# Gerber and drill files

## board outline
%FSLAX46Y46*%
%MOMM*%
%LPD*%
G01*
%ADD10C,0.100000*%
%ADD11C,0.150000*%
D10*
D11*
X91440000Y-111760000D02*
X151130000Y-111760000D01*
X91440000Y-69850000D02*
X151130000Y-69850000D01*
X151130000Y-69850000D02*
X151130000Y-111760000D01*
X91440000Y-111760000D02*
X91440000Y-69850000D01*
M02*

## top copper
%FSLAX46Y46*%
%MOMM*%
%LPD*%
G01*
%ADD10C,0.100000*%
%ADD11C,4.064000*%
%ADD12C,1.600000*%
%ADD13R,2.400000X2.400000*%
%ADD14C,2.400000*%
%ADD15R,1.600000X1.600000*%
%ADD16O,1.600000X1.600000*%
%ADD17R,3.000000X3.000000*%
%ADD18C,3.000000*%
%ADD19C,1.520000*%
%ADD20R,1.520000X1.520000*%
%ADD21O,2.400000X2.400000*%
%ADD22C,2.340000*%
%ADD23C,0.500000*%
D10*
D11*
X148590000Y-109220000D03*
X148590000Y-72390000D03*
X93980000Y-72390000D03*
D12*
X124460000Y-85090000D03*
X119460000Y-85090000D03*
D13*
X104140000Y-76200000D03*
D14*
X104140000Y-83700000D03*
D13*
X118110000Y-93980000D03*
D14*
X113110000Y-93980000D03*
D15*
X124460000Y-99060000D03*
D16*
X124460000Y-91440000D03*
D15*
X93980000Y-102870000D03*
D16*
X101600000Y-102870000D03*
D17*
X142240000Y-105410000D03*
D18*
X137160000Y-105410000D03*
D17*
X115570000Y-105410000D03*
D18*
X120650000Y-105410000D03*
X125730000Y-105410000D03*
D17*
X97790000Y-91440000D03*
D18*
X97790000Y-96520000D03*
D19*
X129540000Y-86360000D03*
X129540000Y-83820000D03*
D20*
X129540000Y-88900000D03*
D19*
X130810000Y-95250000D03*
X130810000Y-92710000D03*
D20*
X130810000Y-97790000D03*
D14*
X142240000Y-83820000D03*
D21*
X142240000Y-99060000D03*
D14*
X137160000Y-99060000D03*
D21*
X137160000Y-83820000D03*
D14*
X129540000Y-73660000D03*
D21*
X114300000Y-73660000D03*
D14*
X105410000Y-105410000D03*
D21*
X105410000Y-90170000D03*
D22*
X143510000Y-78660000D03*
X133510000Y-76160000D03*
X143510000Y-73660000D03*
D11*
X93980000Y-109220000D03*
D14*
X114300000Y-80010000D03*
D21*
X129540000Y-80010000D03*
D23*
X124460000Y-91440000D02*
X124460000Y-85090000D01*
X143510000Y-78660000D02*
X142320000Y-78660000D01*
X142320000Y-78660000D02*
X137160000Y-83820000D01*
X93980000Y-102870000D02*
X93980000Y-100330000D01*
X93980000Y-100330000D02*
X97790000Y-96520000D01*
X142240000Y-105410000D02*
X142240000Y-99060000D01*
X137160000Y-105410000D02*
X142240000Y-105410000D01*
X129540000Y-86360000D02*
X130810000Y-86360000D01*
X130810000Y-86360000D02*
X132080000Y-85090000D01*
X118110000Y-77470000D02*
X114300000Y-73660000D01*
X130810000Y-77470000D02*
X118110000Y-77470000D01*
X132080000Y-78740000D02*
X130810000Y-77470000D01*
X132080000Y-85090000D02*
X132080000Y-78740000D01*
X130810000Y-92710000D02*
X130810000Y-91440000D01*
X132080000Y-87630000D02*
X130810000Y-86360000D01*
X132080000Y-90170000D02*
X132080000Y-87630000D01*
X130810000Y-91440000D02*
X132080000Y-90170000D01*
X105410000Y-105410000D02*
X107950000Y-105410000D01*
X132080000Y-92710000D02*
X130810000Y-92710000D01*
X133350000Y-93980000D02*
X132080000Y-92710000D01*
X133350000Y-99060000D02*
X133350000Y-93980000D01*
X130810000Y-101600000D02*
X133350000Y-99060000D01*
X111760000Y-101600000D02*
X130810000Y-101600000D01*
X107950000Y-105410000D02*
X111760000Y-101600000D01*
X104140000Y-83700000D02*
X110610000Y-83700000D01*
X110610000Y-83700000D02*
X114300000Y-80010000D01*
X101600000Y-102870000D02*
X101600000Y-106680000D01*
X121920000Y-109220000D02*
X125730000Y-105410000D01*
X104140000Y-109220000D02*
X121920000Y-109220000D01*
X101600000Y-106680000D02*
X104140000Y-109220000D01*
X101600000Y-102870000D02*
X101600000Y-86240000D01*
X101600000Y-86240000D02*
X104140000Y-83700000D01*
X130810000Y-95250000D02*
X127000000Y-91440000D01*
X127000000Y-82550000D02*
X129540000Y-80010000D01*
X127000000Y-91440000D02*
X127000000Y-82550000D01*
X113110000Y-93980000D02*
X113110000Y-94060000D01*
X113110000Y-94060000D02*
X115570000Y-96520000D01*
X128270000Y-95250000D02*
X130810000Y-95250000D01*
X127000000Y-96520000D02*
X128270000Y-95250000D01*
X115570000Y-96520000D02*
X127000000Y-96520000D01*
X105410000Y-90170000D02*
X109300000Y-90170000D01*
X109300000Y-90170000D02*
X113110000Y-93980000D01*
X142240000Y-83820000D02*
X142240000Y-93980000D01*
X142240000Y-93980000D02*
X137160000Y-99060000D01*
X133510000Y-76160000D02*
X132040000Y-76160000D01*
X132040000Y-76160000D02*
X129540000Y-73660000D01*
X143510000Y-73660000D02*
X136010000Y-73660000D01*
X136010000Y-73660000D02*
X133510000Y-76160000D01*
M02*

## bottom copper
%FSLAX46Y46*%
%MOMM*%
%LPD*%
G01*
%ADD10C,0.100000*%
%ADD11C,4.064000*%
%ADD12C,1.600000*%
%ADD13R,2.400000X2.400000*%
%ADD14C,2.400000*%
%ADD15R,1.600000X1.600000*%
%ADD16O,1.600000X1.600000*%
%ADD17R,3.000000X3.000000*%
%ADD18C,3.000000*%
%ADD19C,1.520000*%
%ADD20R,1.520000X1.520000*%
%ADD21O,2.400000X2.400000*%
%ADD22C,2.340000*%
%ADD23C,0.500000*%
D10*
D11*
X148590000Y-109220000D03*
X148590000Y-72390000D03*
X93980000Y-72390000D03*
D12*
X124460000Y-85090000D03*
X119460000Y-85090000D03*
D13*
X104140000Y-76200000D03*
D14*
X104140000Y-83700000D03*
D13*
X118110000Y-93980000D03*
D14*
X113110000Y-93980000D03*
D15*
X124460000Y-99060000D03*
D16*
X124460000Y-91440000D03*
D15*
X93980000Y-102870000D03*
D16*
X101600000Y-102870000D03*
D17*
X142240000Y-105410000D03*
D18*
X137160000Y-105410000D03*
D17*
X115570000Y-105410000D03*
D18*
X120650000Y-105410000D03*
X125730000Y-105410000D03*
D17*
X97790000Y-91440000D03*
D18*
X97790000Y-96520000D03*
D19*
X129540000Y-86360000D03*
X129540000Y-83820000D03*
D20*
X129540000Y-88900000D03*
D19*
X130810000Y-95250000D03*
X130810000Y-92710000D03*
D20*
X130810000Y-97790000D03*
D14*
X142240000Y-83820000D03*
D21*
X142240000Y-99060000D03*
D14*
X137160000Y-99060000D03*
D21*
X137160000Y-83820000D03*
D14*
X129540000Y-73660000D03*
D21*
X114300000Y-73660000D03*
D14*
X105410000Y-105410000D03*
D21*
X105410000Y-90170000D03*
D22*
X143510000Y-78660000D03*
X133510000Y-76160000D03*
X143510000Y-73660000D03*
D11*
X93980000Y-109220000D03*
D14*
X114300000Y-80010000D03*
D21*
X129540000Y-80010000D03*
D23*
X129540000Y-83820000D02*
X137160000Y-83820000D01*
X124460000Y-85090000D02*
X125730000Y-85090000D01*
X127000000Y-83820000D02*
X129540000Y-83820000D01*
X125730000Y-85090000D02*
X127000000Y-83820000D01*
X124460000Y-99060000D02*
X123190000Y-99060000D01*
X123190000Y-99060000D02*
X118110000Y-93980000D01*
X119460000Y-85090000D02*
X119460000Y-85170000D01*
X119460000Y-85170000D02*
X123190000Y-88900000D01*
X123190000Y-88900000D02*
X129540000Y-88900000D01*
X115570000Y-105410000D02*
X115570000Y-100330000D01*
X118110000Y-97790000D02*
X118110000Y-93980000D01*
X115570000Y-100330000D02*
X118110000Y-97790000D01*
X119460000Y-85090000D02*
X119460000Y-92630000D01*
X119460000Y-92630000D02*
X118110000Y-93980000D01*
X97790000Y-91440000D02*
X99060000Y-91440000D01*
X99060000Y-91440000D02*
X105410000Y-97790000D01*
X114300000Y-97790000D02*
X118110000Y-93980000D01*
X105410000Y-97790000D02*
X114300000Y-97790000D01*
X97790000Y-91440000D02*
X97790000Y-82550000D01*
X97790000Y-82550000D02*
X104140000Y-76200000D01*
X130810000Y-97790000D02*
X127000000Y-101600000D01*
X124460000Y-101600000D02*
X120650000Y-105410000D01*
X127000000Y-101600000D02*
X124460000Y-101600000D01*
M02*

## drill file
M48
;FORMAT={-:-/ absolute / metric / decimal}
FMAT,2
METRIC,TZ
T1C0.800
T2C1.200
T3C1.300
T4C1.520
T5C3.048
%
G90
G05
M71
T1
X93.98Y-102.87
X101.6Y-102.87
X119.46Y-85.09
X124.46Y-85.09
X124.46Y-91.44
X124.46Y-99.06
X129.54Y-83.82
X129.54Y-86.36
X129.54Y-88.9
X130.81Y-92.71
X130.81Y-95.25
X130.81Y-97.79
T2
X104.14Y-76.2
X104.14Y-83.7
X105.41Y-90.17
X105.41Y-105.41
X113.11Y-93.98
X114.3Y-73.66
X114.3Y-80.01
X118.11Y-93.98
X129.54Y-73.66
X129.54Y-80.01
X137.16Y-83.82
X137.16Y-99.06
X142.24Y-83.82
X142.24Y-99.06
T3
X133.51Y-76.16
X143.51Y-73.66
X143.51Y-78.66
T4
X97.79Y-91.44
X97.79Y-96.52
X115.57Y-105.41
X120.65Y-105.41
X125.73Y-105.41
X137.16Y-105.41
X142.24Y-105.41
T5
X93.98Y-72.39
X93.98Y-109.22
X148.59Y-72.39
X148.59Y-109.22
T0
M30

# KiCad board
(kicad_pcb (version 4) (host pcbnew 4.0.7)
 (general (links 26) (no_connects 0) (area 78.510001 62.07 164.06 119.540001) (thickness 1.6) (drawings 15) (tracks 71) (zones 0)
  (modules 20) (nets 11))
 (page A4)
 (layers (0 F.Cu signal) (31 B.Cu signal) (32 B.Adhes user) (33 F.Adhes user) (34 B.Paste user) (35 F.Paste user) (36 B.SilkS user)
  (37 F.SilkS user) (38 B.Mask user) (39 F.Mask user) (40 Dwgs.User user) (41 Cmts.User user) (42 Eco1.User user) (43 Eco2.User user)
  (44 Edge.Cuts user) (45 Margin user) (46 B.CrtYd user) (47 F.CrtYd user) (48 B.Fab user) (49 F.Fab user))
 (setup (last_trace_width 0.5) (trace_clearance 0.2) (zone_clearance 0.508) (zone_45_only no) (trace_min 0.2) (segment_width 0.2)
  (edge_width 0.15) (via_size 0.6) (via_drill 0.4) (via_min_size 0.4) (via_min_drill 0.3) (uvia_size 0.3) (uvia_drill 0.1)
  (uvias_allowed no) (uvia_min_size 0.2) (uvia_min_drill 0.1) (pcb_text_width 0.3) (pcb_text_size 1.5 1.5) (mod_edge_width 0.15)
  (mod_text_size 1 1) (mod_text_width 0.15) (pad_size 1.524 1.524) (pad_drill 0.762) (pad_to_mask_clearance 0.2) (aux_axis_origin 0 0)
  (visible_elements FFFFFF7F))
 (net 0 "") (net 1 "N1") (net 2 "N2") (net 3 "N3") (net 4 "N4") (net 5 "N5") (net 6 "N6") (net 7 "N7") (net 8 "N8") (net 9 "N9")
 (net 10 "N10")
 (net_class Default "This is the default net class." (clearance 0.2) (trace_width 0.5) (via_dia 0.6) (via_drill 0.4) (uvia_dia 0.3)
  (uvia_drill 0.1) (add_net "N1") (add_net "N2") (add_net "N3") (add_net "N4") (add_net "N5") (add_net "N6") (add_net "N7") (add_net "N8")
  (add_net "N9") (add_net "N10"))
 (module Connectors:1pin (layer F.Cu) (at 148.59 109.22)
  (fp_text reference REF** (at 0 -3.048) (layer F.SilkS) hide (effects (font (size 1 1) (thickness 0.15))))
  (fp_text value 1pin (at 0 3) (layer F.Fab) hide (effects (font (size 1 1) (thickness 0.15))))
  (pad 1 thru_hole circle (at 0 0) (size 4.064 4.064) (drill 3.048) (layers *.Cu *.Mask)))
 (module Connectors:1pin (layer F.Cu) (at 148.59 72.39)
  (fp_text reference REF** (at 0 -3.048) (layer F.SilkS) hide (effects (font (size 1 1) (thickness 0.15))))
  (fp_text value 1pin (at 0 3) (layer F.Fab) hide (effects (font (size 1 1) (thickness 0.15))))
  (pad 1 thru_hole circle (at 0 0) (size 4.064 4.064) (drill 3.048) (layers *.Cu *.Mask)))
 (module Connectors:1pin (layer F.Cu) (at 93.98 72.39)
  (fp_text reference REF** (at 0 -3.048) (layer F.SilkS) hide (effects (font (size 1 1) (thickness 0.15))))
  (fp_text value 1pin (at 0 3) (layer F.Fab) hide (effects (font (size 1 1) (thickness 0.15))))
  (pad 1 thru_hole circle (at 0 0) (size 4.064 4.064) (drill 3.048) (layers *.Cu *.Mask)))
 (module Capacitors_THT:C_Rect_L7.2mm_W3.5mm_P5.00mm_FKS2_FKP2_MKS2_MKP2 (layer F.Cu) (at 124.46 85.09 180)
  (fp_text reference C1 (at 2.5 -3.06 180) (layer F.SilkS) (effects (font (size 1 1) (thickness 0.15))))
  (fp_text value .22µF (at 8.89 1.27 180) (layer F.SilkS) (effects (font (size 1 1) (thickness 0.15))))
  (pad 1 thru_hole circle (at 0 0 180) (size 1.6 1.6) (drill 0.8) (layers *.Cu *.Mask) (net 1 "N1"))
  (pad 2 thru_hole circle (at 5 0 180) (size 1.6 1.6) (drill 0.8) (layers *.Cu *.Mask) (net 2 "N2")))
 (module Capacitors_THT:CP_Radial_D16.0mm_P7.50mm (layer F.Cu) (at 104.14 76.2 270)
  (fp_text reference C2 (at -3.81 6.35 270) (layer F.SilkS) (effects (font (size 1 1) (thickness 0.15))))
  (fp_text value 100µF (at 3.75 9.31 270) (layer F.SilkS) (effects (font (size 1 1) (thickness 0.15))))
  (pad 1 thru_hole rect (at 0 0 270) (size 2.4 2.4) (drill 1.2) (layers *.Cu *.Mask) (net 2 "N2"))
  (pad 2 thru_hole circle (at 7.5 0 270) (size 2.4 2.4) (drill 1.2) (layers *.Cu *.Mask) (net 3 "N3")))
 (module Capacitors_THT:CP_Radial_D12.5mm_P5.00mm (layer F.Cu) (at 118.11 93.98 180)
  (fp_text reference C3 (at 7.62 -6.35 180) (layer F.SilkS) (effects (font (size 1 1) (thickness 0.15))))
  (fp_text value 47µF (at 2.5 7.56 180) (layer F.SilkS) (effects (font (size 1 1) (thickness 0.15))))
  (pad 1 thru_hole rect (at 0 0 180) (size 2.4 2.4) (drill 1.2) (layers *.Cu *.Mask) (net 2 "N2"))
  (pad 2 thru_hole circle (at 5 0 180) (size 2.4 2.4) (drill 1.2) (layers *.Cu *.Mask) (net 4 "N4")))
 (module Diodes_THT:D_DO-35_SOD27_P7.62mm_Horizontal (layer F.Cu) (at 124.46 99.06 90)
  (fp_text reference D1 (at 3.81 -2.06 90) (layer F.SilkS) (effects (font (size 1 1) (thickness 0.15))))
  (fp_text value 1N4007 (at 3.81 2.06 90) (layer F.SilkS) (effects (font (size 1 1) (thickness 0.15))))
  (pad 1 thru_hole rect (at 0 0 90) (size 1.6 1.6) (drill 0.8) (layers *.Cu *.Mask) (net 2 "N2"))
  (pad 2 thru_hole oval (at 7.62 0 90) (size 1.6 1.6) (drill 0.8) (layers *.Cu *.Mask) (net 1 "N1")))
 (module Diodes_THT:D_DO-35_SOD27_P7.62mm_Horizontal (layer F.Cu) (at 93.98 102.87)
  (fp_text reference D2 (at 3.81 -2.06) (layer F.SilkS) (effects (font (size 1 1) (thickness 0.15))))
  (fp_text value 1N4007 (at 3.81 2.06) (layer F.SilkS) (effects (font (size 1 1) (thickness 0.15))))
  (pad 1 thru_hole rect (at 0 0) (size 1.6 1.6) (drill 0.8) (layers *.Cu *.Mask) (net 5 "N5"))
  (pad 2 thru_hole oval (at 7.62 0) (size 1.6 1.6) (drill 0.8) (layers *.Cu *.Mask) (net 3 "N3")))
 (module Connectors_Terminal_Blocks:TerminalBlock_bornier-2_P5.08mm (layer F.Cu) (at 142.24 105.41 180)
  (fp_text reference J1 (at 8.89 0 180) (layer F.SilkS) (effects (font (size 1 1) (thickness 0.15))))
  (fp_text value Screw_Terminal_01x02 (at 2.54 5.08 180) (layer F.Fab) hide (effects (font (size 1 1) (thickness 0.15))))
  (pad 1 thru_hole rect (at 0 0 180) (size 3 3) (drill 1.52) (layers *.Cu *.Mask) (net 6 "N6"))
  (pad 2 thru_hole circle (at 5.08 0 180) (size 3 3) (drill 1.52) (layers *.Cu *.Mask) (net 6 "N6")))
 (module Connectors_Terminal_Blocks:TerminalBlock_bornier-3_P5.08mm (layer F.Cu) (at 115.57 105.41)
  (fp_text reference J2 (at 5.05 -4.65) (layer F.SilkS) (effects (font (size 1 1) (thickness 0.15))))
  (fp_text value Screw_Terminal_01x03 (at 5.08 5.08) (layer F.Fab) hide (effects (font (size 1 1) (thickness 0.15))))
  (pad 1 thru_hole rect (at 0 0) (size 3 3) (drill 1.52) (layers *.Cu *.Mask) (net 2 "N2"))
  (pad 2 thru_hole circle (at 5.08 0) (size 3 3) (drill 1.52) (layers *.Cu *.Mask) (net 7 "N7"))
  (pad 3 thru_hole circle (at 10.16 0) (size 3 3) (drill 1.52) (layers *.Cu *.Mask) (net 3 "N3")))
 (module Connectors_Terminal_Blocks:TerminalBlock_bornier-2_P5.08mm (layer F.Cu) (at 97.79 91.44 270)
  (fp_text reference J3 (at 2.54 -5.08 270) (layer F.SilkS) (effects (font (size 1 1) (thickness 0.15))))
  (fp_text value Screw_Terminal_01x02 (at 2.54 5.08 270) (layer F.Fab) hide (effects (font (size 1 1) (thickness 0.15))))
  (pad 1 thru_hole rect (at 0 0 270) (size 3 3) (drill 1.52) (layers *.Cu *.Mask) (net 2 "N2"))
  (pad 2 thru_hole circle (at 5.08 0 270) (size 3 3) (drill 1.52) (layers *.Cu *.Mask) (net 5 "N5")))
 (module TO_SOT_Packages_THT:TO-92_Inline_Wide (layer F.Cu) (at 129.54 88.9 90)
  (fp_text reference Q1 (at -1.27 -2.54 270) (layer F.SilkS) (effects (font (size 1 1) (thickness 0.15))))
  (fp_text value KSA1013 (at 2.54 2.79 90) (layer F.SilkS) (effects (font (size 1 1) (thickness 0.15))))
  (pad 2 thru_hole circle (at 2.54 0 180) (size 1.52 1.52) (drill 0.8) (layers *.Cu *.Mask) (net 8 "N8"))
  (pad 3 thru_hole circle (at 5.08 0 180) (size 1.52 1.52) (drill 0.8) (layers *.Cu *.Mask) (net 1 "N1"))
  (pad 1 thru_hole rect (at 0 0 180) (size 1.52 1.52) (drill 0.8) (layers *.Cu *.Mask) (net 2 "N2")))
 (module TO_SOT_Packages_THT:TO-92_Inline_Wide (layer F.Cu) (at 130.81 97.79 90)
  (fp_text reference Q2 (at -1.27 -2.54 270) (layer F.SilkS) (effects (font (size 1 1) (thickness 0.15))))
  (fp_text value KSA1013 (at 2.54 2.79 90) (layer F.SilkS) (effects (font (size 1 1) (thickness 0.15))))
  (pad 2 thru_hole circle (at 2.54 0 180) (size 1.52 1.52) (drill 0.8) (layers *.Cu *.Mask) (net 4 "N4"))
  (pad 3 thru_hole circle (at 5.08 0 180) (size 1.52 1.52) (drill 0.8) (layers *.Cu *.Mask) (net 8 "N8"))
  (pad 1 thru_hole rect (at 0 0 180) (size 1.52 1.52) (drill 0.8) (layers *.Cu *.Mask) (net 7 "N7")))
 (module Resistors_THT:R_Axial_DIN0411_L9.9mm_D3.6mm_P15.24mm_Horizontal (layer F.Cu) (at 142.24 83.82 270)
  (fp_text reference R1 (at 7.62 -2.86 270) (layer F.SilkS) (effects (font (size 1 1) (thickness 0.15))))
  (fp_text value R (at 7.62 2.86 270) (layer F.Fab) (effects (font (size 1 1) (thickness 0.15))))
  (pad 1 thru_hole circle (at 0 0 270) (size 2.4 2.4) (drill 1.2) (layers *.Cu *.Mask) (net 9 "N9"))
  (pad 2 thru_hole oval (at 15.24 0 270) (size 2.4 2.4) (drill 1.2) (layers *.Cu *.Mask) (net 6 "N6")))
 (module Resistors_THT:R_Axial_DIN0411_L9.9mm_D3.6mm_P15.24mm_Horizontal (layer F.Cu) (at 137.16 99.06 90)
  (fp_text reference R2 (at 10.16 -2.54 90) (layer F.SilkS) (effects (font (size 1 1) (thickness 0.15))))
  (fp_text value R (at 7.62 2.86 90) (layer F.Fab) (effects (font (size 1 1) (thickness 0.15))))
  (pad 1 thru_hole circle (at 0 0 90) (size 2.4 2.4) (drill 1.2) (layers *.Cu *.Mask) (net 9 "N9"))
  (pad 2 thru_hole oval (at 15.24 0 90) (size 2.4 2.4) (drill 1.2) (layers *.Cu *.Mask) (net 1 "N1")))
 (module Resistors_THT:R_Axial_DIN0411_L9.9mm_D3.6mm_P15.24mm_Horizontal (layer F.Cu) (at 129.54 73.66 180)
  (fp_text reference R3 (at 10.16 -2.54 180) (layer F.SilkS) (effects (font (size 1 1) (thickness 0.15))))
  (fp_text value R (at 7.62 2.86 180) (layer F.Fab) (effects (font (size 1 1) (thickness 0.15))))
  (pad 1 thru_hole circle (at 0 0 180) (size 2.4 2.4) (drill 1.2) (layers *.Cu *.Mask) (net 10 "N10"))
  (pad 2 thru_hole oval (at 15.24 0 180) (size 2.4 2.4) (drill 1.2) (layers *.Cu *.Mask) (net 8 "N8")))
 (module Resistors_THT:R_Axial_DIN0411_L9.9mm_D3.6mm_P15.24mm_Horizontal (layer F.Cu) (at 105.41 105.41 90)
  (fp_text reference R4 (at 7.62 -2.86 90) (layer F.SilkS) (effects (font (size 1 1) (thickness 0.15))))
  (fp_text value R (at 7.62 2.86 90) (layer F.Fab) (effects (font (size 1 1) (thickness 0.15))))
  (pad 1 thru_hole circle (at 0 0 90) (size 2.4 2.4) (drill 1.2) (layers *.Cu *.Mask) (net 8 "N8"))
  (pad 2 thru_hole oval (at 15.24 0 90) (size 2.4 2.4) (drill 1.2) (layers *.Cu *.Mask) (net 4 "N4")))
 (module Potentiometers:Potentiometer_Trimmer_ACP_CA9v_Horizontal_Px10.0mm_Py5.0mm (layer F.Cu) (at 143.51 73.66 180)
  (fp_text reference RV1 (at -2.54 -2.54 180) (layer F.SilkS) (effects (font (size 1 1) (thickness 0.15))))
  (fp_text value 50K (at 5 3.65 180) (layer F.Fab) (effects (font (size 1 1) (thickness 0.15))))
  (pad 3 thru_hole circle (at 0 -5 180) (size 2.34 2.34) (drill 1.3) (layers *.Cu *.Mask) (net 1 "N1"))
  (pad 2 thru_hole circle (at 10 -2.5 180) (size 2.34 2.34) (drill 1.3) (layers *.Cu *.Mask) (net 10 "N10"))
  (pad 1 thru_hole circle (at 0 0 180) (size 2.34 2.34) (drill 1.3) (layers *.Cu *.Mask) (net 10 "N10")))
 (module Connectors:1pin (layer F.Cu) (at 93.98 109.22)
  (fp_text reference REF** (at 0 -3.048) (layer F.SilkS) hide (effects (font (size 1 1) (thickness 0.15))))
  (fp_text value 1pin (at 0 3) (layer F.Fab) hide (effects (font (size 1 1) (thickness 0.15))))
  (pad 1 thru_hole circle (at 0 0) (size 4.064 4.064) (drill 3.048) (layers *.Cu *.Mask)))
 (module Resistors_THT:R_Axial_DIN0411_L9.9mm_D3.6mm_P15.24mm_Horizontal (layer F.Cu) (at 114.3 80.01)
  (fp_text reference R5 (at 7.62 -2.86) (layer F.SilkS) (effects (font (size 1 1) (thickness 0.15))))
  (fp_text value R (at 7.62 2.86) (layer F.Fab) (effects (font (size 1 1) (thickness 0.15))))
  (pad 1 thru_hole circle (at 0 0) (size 2.4 2.4) (drill 1.2) (layers *.Cu *.Mask) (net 3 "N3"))
  (pad 2 thru_hole oval (at 15.24 0) (size 2.4 2.4) (drill 1.2) (layers *.Cu *.Mask) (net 4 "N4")))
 (gr_line (start 91.44 111.76) (end 151.13 111.76) (angle 90) (layer Edge.Cuts) (width 0.15))
 (gr_line (start 91.44 69.85) (end 151.13 69.85) (angle 90) (layer Edge.Cuts) (width 0.15))
 (gr_line (start 151.13 69.85) (end 151.13 111.76) (angle 90) (layer Edge.Cuts) (width 0.15))
 (gr_line (start 91.44 111.76) (end 91.44 69.85) (angle 90) (layer Edge.Cuts) (width 0.15))
 (segment (start 124.46 91.44) (end 124.46 85.09) (width 0.5) (layer F.Cu) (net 1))
 (segment (start 129.54 83.82) (end 137.16 83.82) (width 0.5) (layer B.Cu) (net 1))
 (segment (start 124.46 85.09) (end 125.73 85.09) (width 0.5) (layer B.Cu) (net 1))
 (segment (start 127 83.82) (end 129.54 83.82) (width 0.5) (layer B.Cu) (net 1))
 (segment (start 125.73 85.09) (end 127 83.82) (width 0.5) (layer B.Cu) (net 1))
 (segment (start 143.51 78.66) (end 142.32 78.66) (width 0.5) (layer F.Cu) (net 1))
 (segment (start 142.32 78.66) (end 137.16 83.82) (width 0.5) (layer F.Cu) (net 1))
 (segment (start 124.46 99.06) (end 123.19 99.06) (width 0.5) (layer B.Cu) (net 2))
 (segment (start 123.19 99.06) (end 118.11 93.98) (width 0.5) (layer B.Cu) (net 2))
 (segment (start 119.46 85.09) (end 119.46 85.17) (width 0.5) (layer B.Cu) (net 2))
 (segment (start 119.46 85.17) (end 123.19 88.9) (width 0.5) (layer B.Cu) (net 2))
 (segment (start 123.19 88.9) (end 129.54 88.9) (width 0.5) (layer B.Cu) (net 2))
 (segment (start 115.57 105.41) (end 115.57 100.33) (width 0.5) (layer B.Cu) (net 2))
 (segment (start 118.11 97.79) (end 118.11 93.98) (width 0.5) (layer B.Cu) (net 2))
 (segment (start 115.57 100.33) (end 118.11 97.79) (width 0.5) (layer B.Cu) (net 2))
 (segment (start 119.46 85.09) (end 119.46 92.63) (width 0.5) (layer B.Cu) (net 2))
 (segment (start 119.46 92.63) (end 118.11 93.98) (width 0.5) (layer B.Cu) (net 2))
 (segment (start 97.79 91.44) (end 99.06 91.44) (width 0.5) (layer B.Cu) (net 2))
 (segment (start 99.06 91.44) (end 105.41 97.79) (width 0.5) (layer B.Cu) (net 2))
 (segment (start 114.3 97.79) (end 118.11 93.98) (width 0.5) (layer B.Cu) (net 2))
 (segment (start 105.41 97.79) (end 114.3 97.79) (width 0.5) (layer B.Cu) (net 2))
 (segment (start 97.79 91.44) (end 97.79 82.55) (width 0.5) (layer B.Cu) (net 2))
 (segment (start 97.79 82.55) (end 104.14 76.2) (width 0.5) (layer B.Cu) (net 2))
 (segment (start 93.98 102.87) (end 93.98 100.33) (width 0.5) (layer F.Cu) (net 5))
 (segment (start 93.98 100.33) (end 97.79 96.52) (width 0.5) (layer F.Cu) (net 5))
 (segment (start 142.24 105.41) (end 142.24 99.06) (width 0.5) (layer F.Cu) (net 6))
 (segment (start 137.16 105.41) (end 142.24 105.41) (width 0.5) (layer F.Cu) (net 6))
 (segment (start 130.81 97.79) (end 127 101.6) (width 0.5) (layer B.Cu) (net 7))
 (segment (start 124.46 101.6) (end 120.65 105.41) (width 0.5) (layer B.Cu) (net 7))
 (segment (start 127 101.6) (end 124.46 101.6) (width 0.5) (layer B.Cu) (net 7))
 (segment (start 129.54 86.36) (end 130.81 86.36) (width 0.5) (layer F.Cu) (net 8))
 (segment (start 130.81 86.36) (end 132.08 85.09) (width 0.5) (layer F.Cu) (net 8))
 (segment (start 118.11 77.47) (end 114.3 73.66) (width 0.5) (layer F.Cu) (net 8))
 (segment (start 130.81 77.47) (end 118.11 77.47) (width 0.5) (layer F.Cu) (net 8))
 (segment (start 132.08 78.74) (end 130.81 77.47) (width 0.5) (layer F.Cu) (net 8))
 (segment (start 132.08 85.09) (end 132.08 78.74) (width 0.5) (layer F.Cu) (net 8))
 (segment (start 130.81 92.71) (end 130.81 91.44) (width 0.5) (layer F.Cu) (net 8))
 (segment (start 132.08 87.63) (end 130.81 86.36) (width 0.5) (layer F.Cu) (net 8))
 (segment (start 132.08 90.17) (end 132.08 87.63) (width 0.5) (layer F.Cu) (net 8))
 (segment (start 130.81 91.44) (end 132.08 90.17) (width 0.5) (layer F.Cu) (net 8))
 (segment (start 105.41 105.41) (end 107.95 105.41) (width 0.5) (layer F.Cu) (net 8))
 (segment (start 132.08 92.71) (end 130.81 92.71) (width 0.5) (layer F.Cu) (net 8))
 (segment (start 133.35 93.98) (end 132.08 92.71) (width 0.5) (layer F.Cu) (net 8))
 (segment (start 133.35 99.06) (end 133.35 93.98) (width 0.5) (layer F.Cu) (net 8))
 (segment (start 130.81 101.6) (end 133.35 99.06) (width 0.5) (layer F.Cu) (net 8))
 (segment (start 111.76 101.6) (end 130.81 101.6) (width 0.5) (layer F.Cu) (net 8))
 (segment (start 107.95 105.41) (end 111.76 101.6) (width 0.5) (layer F.Cu) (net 8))
 (segment (start 104.14 83.7) (end 110.61 83.7) (width 0.5) (layer F.Cu) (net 3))
 (segment (start 110.61 83.7) (end 114.3 80.01) (width 0.5) (layer F.Cu) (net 3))
 (segment (start 101.6 102.87) (end 101.6 106.68) (width 0.5) (layer F.Cu) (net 3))
 (segment (start 121.92 109.22) (end 125.73 105.41) (width 0.5) (layer F.Cu) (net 3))
 (segment (start 104.14 109.22) (end 121.92 109.22) (width 0.5) (layer F.Cu) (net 3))
 (segment (start 101.6 106.68) (end 104.14 109.22) (width 0.5) (layer F.Cu) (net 3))
 (segment (start 101.6 102.87) (end 101.6 86.24) (width 0.5) (layer F.Cu) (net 3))
 (segment (start 101.6 86.24) (end 104.14 83.7) (width 0.5) (layer F.Cu) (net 3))
 (segment (start 130.81 95.25) (end 127 91.44) (width 0.5) (layer F.Cu) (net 4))
 (segment (start 127 82.55) (end 129.54 80.01) (width 0.5) (layer F.Cu) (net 4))
 (segment (start 127 91.44) (end 127 82.55) (width 0.5) (layer F.Cu) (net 4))
 (segment (start 113.11 93.98) (end 113.11 94.06) (width 0.5) (layer F.Cu) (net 4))
 (segment (start 113.11 94.06) (end 115.57 96.52) (width 0.5) (layer F.Cu) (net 4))
 (segment (start 128.27 95.25) (end 130.81 95.25) (width 0.5) (layer F.Cu) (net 4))
 (segment (start 127 96.52) (end 128.27 95.25) (width 0.5) (layer F.Cu) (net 4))
 (segment (start 115.57 96.52) (end 127 96.52) (width 0.5) (layer F.Cu) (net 4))
 (segment (start 105.41 90.17) (end 109.3 90.17) (width 0.5) (layer F.Cu) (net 4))
 (segment (start 109.3 90.17) (end 113.11 93.98) (width 0.5) (layer F.Cu) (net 4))
 (segment (start 142.24 83.82) (end 142.24 93.98) (width 0.5) (layer F.Cu) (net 9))
 (segment (start 142.24 93.98) (end 137.16 99.06) (width 0.5) (layer F.Cu) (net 9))
 (segment (start 133.51 76.16) (end 132.04 76.16) (width 0.5) (layer F.Cu) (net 10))
 (segment (start 132.04 76.16) (end 129.54 73.66) (width 0.5) (layer F.Cu) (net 10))
 (segment (start 143.51 73.66) (end 136.01 73.66) (width 0.5) (layer F.Cu) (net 10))
 (segment (start 136.01 73.66) (end 133.51 76.16) (width 0.5) (layer F.Cu) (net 10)))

